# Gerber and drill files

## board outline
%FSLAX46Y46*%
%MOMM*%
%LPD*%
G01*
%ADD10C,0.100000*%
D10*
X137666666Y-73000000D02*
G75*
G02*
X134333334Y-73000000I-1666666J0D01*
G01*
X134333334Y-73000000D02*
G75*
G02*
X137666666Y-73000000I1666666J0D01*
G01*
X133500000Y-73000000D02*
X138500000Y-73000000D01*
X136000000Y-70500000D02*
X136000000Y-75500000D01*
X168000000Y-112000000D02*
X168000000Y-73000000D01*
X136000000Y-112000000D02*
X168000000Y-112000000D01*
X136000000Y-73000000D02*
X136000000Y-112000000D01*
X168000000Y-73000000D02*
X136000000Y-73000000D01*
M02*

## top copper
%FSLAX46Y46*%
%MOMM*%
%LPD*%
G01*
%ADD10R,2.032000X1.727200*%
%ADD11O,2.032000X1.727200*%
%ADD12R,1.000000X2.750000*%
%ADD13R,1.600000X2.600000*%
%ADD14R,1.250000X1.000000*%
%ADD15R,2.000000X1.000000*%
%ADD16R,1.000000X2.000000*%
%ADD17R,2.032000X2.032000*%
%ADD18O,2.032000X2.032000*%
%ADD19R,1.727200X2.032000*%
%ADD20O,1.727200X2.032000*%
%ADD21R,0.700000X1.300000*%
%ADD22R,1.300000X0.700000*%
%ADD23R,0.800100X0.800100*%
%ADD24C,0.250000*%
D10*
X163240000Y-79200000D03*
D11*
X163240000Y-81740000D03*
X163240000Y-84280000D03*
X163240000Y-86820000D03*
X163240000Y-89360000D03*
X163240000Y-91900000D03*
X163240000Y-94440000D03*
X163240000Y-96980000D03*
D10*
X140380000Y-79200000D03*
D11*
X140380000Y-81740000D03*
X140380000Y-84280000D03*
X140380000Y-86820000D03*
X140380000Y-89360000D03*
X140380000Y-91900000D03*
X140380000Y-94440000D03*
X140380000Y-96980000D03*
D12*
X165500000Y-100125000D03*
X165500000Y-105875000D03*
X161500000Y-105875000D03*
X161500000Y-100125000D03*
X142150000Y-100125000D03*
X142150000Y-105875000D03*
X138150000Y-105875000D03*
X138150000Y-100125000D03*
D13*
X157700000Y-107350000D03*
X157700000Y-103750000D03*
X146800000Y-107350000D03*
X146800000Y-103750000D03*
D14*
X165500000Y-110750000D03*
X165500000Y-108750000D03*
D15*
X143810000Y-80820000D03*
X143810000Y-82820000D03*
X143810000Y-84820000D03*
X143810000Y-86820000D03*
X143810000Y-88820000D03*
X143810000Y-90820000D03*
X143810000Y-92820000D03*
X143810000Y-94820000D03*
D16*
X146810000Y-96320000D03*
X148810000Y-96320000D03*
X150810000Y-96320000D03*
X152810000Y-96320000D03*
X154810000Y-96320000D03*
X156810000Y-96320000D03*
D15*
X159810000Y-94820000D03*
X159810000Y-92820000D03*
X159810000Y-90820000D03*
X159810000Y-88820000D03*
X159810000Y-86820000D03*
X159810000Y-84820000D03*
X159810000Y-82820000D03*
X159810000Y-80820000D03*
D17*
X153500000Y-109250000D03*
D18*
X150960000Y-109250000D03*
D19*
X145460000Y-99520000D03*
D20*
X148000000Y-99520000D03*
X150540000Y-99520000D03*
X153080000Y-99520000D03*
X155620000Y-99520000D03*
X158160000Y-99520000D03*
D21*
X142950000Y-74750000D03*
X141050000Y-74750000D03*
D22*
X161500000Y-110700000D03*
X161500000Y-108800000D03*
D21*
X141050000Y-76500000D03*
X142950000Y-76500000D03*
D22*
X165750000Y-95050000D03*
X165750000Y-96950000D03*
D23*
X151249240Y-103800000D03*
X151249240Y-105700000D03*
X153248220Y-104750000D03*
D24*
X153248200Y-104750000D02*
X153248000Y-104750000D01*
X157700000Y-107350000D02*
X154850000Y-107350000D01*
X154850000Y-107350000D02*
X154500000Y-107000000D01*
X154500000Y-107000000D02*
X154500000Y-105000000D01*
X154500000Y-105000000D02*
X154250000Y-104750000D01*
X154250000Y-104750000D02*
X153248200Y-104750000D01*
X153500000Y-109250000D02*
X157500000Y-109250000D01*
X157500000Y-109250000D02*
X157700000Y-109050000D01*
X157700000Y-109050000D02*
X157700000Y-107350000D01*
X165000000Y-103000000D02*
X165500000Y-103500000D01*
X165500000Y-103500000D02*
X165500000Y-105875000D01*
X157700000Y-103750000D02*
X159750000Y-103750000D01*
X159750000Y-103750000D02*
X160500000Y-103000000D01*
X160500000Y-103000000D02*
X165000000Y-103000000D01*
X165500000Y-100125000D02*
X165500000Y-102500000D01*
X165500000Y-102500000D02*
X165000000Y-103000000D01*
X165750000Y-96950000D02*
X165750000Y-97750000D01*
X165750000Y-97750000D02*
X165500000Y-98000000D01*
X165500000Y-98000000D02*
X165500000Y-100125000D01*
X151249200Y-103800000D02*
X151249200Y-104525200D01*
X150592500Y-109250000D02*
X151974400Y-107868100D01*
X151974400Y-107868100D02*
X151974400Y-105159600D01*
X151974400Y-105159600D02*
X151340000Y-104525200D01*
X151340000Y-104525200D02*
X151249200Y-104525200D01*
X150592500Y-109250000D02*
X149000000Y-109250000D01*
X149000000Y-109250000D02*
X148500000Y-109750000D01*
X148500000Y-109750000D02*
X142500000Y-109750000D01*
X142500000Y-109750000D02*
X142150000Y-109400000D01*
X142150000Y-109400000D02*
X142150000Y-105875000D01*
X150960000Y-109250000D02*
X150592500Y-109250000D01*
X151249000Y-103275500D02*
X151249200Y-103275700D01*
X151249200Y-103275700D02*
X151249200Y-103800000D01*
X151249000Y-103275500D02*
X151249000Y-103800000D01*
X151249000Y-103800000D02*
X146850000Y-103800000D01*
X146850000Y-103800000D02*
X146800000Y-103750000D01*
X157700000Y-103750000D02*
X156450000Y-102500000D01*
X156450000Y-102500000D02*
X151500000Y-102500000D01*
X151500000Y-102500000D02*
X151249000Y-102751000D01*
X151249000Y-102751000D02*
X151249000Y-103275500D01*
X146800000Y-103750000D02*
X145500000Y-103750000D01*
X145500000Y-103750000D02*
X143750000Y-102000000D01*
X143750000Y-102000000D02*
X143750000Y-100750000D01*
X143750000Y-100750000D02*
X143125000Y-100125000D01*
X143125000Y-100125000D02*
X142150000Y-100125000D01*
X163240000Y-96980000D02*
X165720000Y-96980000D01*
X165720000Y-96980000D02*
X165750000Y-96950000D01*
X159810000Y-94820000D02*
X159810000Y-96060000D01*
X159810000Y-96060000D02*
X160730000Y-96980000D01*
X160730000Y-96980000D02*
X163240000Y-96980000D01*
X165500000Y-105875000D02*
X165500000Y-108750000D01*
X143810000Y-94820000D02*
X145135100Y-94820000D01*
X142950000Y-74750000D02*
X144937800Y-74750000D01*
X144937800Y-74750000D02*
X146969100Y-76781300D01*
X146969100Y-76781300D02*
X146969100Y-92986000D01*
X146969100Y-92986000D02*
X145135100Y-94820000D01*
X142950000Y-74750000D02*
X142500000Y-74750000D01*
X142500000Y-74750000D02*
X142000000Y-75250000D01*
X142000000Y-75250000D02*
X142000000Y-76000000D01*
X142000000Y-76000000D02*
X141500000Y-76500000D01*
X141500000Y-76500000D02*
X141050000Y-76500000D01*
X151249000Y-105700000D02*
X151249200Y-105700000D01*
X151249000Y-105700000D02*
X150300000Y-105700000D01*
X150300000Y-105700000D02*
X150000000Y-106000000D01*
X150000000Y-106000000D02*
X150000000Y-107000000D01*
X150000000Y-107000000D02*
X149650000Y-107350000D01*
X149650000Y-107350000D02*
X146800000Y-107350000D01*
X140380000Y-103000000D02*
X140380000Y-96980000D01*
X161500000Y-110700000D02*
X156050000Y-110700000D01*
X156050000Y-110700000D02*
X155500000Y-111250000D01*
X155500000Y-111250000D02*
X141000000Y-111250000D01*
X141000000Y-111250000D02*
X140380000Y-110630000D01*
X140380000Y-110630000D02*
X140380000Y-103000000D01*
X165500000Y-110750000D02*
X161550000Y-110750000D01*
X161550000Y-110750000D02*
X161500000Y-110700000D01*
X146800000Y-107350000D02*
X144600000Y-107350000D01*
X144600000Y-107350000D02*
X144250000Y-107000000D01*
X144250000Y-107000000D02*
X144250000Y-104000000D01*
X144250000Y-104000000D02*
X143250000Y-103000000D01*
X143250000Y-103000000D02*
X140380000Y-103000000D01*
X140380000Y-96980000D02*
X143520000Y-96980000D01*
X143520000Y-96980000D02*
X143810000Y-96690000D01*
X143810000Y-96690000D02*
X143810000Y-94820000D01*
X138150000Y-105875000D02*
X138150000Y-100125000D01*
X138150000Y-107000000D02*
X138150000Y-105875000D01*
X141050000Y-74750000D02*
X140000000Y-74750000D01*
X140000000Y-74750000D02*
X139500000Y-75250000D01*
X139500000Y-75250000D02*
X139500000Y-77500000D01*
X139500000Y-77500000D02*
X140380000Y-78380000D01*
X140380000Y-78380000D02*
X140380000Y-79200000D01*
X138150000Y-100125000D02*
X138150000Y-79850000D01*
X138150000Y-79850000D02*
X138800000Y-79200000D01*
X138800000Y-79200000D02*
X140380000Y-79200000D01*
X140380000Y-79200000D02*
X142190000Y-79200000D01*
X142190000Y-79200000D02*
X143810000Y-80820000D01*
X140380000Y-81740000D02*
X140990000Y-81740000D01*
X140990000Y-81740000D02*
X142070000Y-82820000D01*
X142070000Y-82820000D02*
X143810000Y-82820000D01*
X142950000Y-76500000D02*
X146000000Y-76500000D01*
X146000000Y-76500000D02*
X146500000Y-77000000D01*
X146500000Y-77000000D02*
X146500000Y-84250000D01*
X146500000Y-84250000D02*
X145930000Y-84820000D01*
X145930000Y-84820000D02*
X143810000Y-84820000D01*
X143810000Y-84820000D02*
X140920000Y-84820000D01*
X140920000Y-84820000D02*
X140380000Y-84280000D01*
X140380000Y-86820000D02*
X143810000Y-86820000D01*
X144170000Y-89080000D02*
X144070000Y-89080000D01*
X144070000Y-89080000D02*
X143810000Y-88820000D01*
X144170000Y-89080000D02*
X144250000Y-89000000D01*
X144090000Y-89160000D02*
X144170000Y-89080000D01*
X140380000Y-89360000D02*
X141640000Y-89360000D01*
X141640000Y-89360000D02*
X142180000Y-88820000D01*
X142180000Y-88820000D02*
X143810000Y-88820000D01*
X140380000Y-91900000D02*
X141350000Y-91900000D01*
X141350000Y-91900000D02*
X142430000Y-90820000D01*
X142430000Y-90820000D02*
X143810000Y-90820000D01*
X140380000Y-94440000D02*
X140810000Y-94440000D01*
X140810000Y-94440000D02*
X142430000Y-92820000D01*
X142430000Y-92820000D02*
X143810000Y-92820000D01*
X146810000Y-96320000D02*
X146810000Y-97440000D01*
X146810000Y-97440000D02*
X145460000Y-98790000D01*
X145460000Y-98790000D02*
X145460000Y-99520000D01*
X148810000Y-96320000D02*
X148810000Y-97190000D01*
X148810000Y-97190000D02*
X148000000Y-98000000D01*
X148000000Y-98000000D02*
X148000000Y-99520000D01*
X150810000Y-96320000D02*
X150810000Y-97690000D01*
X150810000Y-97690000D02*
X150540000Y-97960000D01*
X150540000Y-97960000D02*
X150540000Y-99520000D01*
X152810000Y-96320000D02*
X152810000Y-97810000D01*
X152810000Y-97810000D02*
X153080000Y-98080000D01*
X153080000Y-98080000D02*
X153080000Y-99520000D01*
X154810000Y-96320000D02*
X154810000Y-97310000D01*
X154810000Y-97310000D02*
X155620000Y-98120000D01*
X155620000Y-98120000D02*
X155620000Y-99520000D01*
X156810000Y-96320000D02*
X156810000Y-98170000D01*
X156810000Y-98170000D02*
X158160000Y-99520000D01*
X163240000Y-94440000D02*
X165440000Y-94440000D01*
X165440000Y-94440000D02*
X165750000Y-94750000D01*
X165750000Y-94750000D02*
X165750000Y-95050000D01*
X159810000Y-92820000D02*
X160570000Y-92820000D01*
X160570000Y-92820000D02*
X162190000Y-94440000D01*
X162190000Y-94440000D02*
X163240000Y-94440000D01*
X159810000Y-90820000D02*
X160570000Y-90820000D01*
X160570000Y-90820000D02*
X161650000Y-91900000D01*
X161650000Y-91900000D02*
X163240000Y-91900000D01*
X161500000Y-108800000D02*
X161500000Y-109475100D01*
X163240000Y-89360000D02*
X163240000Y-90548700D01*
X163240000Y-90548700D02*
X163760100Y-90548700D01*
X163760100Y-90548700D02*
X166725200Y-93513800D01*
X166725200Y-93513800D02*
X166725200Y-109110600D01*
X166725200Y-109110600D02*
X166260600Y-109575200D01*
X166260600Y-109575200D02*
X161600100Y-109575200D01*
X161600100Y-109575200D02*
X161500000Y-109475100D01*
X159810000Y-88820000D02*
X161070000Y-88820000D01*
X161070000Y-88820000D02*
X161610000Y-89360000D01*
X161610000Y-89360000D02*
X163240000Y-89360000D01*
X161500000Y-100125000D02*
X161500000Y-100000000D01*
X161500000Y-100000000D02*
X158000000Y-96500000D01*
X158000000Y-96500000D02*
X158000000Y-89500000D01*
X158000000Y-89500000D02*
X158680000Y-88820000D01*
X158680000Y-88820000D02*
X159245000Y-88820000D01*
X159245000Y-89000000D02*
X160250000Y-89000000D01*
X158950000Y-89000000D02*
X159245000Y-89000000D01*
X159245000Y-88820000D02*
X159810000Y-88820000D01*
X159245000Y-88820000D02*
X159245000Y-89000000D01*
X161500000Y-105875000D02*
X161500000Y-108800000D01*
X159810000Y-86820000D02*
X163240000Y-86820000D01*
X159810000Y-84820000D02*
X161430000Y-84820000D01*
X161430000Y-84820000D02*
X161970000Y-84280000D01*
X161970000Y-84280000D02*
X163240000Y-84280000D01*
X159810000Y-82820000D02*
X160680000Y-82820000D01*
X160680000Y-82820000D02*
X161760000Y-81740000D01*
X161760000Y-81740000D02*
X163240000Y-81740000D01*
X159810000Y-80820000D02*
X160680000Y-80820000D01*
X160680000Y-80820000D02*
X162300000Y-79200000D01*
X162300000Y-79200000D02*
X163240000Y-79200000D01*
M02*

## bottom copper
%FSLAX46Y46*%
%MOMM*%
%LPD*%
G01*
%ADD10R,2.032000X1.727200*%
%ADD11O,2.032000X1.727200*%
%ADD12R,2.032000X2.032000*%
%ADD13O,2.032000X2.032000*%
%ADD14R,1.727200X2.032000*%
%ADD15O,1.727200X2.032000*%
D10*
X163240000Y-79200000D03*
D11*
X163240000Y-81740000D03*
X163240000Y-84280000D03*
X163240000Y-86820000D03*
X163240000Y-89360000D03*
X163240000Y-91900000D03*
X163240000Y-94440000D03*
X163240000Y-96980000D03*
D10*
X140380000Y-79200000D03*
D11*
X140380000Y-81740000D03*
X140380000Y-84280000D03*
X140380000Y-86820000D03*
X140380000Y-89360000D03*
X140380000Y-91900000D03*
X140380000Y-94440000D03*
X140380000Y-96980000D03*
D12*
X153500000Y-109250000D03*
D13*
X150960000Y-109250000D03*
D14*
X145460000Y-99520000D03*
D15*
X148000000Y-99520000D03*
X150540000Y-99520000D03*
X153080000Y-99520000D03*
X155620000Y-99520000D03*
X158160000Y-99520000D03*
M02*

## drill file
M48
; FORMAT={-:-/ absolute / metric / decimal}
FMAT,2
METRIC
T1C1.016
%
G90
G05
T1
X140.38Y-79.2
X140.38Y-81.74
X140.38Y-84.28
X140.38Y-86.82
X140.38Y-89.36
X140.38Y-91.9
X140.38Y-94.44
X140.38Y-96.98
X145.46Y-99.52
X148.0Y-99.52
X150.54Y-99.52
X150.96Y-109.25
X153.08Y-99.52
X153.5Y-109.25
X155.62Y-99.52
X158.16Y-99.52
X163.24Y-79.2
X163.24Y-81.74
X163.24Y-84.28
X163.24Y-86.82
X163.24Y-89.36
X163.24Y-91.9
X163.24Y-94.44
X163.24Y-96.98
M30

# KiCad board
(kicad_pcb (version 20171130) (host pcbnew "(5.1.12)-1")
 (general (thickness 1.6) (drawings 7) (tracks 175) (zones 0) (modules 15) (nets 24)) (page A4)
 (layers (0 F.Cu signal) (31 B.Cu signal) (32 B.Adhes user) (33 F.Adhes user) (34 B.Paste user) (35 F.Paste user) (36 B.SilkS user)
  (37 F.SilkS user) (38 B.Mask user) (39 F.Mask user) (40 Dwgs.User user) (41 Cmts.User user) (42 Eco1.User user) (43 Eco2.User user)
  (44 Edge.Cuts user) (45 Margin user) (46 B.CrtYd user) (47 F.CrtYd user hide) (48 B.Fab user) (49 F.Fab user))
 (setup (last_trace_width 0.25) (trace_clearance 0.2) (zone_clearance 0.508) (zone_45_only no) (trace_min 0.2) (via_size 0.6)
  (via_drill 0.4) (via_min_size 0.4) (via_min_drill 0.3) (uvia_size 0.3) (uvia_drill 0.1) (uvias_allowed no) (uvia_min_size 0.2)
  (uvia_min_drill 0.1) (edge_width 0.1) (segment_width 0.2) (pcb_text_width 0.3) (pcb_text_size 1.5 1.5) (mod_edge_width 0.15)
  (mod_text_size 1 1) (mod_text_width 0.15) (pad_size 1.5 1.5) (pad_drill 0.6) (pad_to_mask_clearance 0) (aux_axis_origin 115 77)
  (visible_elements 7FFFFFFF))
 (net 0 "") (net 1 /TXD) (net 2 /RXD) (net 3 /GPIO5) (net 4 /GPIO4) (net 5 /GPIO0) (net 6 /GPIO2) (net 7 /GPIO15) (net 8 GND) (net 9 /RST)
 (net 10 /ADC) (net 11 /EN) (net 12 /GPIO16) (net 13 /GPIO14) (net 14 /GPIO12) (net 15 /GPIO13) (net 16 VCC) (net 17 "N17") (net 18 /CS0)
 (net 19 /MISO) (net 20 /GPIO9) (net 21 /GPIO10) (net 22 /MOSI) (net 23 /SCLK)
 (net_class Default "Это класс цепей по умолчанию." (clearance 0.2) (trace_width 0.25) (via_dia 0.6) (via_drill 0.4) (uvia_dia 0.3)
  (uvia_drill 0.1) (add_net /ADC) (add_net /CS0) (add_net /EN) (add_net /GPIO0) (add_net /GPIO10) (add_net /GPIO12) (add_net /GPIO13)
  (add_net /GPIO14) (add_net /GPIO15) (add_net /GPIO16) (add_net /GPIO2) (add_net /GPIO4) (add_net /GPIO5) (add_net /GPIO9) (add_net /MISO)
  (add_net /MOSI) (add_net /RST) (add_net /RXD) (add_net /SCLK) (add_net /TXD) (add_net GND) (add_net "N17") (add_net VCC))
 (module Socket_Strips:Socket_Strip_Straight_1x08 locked (layer F.Cu) (at 163.24 79.2 270)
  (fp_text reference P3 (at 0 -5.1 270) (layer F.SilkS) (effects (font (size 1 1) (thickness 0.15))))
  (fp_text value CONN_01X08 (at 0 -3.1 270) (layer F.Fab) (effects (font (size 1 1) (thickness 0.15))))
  (pad 1 thru_hole rect (at 0 0 270) (size 1.7272 2.032) (drill 1.016) (layers *.Cu *.Mask F.SilkS) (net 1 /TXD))
  (pad 2 thru_hole oval (at 2.54 0 270) (size 1.7272 2.032) (drill 1.016) (layers *.Cu *.Mask F.SilkS) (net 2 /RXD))
  (pad 3 thru_hole oval (at 5.08 0 270) (size 1.7272 2.032) (drill 1.016) (layers *.Cu *.Mask F.SilkS) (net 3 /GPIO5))
  (pad 4 thru_hole oval (at 7.62 0 270) (size 1.7272 2.032) (drill 1.016) (layers *.Cu *.Mask F.SilkS) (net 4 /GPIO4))
  (pad 5 thru_hole oval (at 10.16 0 270) (size 1.7272 2.032) (drill 1.016) (layers *.Cu *.Mask F.SilkS) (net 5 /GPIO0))
  (pad 6 thru_hole oval (at 12.7 0 270) (size 1.7272 2.032) (drill 1.016) (layers *.Cu *.Mask F.SilkS) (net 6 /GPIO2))
  (pad 7 thru_hole oval (at 15.24 0 270) (size 1.7272 2.032) (drill 1.016) (layers *.Cu *.Mask F.SilkS) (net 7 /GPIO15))
  (pad 8 thru_hole oval (at 17.78 0 270) (size 1.7272 2.032) (drill 1.016) (layers *.Cu *.Mask F.SilkS) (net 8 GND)))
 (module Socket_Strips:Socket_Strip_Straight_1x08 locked (layer F.Cu) (at 140.38 79.2 270)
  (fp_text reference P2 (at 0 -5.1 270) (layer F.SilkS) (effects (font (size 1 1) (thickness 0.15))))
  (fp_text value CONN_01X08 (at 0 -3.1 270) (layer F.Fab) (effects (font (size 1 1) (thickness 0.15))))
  (pad 1 thru_hole rect (at 0 0 270) (size 1.7272 2.032) (drill 1.016) (layers *.Cu *.Mask F.SilkS) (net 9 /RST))
  (pad 2 thru_hole oval (at 2.54 0 270) (size 1.7272 2.032) (drill 1.016) (layers *.Cu *.Mask F.SilkS) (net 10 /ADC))
  (pad 3 thru_hole oval (at 5.08 0 270) (size 1.7272 2.032) (drill 1.016) (layers *.Cu *.Mask F.SilkS) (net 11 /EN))
  (pad 4 thru_hole oval (at 7.62 0 270) (size 1.7272 2.032) (drill 1.016) (layers *.Cu *.Mask F.SilkS) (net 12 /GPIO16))
  (pad 5 thru_hole oval (at 10.16 0 270) (size 1.7272 2.032) (drill 1.016) (layers *.Cu *.Mask F.SilkS) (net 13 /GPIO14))
  (pad 6 thru_hole oval (at 12.7 0 270) (size 1.7272 2.032) (drill 1.016) (layers *.Cu *.Mask F.SilkS) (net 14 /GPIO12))
  (pad 7 thru_hole oval (at 15.24 0 270) (size 1.7272 2.032) (drill 1.016) (layers *.Cu *.Mask F.SilkS) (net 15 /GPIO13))
  (pad 8 thru_hole oval (at 17.78 0 270) (size 1.7272 2.032) (drill 1.016) (layers *.Cu *.Mask F.SilkS) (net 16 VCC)))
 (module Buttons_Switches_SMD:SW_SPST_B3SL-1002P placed (layer F.Cu) (at 163.5 103 270)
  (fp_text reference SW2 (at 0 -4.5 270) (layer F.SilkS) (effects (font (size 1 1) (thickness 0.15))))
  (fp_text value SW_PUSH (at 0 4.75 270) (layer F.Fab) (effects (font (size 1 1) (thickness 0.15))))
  (pad 1 smd rect (at -2.875 -2 270) (size 2.75 1) (layers F.Cu F.Paste F.Mask) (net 8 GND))
  (pad 1 smd rect (at 2.875 -2 270) (size 2.75 1) (layers F.Cu F.Paste F.Mask) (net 8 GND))
  (pad 2 smd rect (at 2.875 2 270) (size 2.75 1) (layers F.Cu F.Paste F.Mask) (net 5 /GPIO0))
  (pad 2 smd rect (at -2.875 2 270) (size 2.75 1) (layers F.Cu F.Paste F.Mask) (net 5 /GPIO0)))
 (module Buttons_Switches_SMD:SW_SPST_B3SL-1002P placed (layer F.Cu) (at 140.15 103 270)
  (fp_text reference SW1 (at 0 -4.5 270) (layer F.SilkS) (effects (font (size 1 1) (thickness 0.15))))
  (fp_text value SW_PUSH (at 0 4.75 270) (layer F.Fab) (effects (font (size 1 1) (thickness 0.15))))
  (pad 1 smd rect (at -2.875 -2 270) (size 2.75 1) (layers F.Cu F.Paste F.Mask) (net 8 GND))
  (pad 1 smd rect (at 2.875 -2 270) (size 2.75 1) (layers F.Cu F.Paste F.Mask) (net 8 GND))
  (pad 2 smd rect (at 2.875 2 270) (size 2.75 1) (layers F.Cu F.Paste F.Mask) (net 9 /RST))
  (pad 2 smd rect (at -2.875 2 270) (size 2.75 1) (layers F.Cu F.Paste F.Mask) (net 9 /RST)))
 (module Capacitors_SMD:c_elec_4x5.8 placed (layer F.Cu) (at 157.7 105.55 90)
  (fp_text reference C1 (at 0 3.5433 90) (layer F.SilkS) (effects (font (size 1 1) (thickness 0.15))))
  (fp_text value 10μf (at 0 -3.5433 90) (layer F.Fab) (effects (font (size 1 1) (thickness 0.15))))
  (pad 1 smd rect (at -1.8 0 270) (size 2.6 1.6) (layers F.Cu F.Paste F.Mask) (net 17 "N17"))
  (pad 2 smd rect (at 1.8 0 270) (size 2.6 1.6) (layers F.Cu F.Paste F.Mask) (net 8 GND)))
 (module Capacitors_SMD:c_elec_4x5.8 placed (layer F.Cu) (at 146.8 105.55 90)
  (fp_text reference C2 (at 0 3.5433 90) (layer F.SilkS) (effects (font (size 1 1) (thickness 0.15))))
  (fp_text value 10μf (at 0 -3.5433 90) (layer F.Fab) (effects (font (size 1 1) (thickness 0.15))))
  (pad 1 smd rect (at -1.8 0 270) (size 2.6 1.6) (layers F.Cu F.Paste F.Mask) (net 16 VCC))
  (pad 2 smd rect (at 1.8 0 270) (size 2.6 1.6) (layers F.Cu F.Paste F.Mask) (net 8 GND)))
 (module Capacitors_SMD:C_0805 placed (layer F.Cu) (at 165.5 109.75 90)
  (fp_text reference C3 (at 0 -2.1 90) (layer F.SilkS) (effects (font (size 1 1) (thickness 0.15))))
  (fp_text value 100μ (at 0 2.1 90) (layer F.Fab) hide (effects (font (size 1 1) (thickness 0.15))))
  (pad 1 smd rect (at -1 0 90) (size 1 1.25) (layers F.Cu F.Paste F.Mask) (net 16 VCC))
  (pad 2 smd rect (at 1 0 90) (size 1 1.25) (layers F.Cu F.Paste F.Mask) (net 8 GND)))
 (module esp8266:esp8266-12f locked (layer F.Cu) (at 151.81 86.82)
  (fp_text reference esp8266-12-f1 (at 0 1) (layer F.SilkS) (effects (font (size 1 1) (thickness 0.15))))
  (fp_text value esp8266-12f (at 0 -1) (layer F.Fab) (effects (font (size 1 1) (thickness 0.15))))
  (pad 1 smd rect (at -8 -6) (size 2 1) (layers F.Cu F.Paste F.Mask) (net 9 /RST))
  (pad 2 smd rect (at -8 -4) (size 2 1) (layers F.Cu F.Paste F.Mask) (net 10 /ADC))
  (pad 3 smd rect (at -8 -2) (size 2 1) (layers F.Cu F.Paste F.Mask) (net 11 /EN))
  (pad 4 smd rect (at -8 0) (size 2 1) (layers F.Cu F.Paste F.Mask) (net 12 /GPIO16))
  (pad 5 smd rect (at -8 2) (size 2 1) (layers F.Cu F.Paste F.Mask) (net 13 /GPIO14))
  (pad 6 smd rect (at -8 4) (size 2 1) (layers F.Cu F.Paste F.Mask) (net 14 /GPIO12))
  (pad 7 smd rect (at -8 6) (size 2 1) (layers F.Cu F.Paste F.Mask) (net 15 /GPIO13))
  (pad 8 smd rect (at -8 8) (size 2 1) (layers F.Cu F.Paste F.Mask) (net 16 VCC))
  (pad 9 smd rect (at -5 9.5) (size 1 2) (layers F.Cu F.Paste F.Mask) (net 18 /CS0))
  (pad 10 smd rect (at -3 9.5) (size 1 2) (layers F.Cu F.Paste F.Mask) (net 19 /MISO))
  (pad 11 smd rect (at -1 9.5) (size 1 2) (layers F.Cu F.Paste F.Mask) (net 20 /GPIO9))
  (pad 12 smd rect (at 1 9.5) (size 1 2) (layers F.Cu F.Paste F.Mask) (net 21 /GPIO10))
  (pad 13 smd rect (at 3 9.5) (size 1 2) (layers F.Cu F.Paste F.Mask) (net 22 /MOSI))
  (pad 14 smd rect (at 5 9.5) (size 1 2) (layers F.Cu F.Paste F.Mask) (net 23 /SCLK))
  (pad 15 smd rect (at 8 8) (size 2 1) (layers F.Cu F.Paste F.Mask) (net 8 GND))
  (pad 16 smd rect (at 8 6) (size 2 1) (layers F.Cu F.Paste F.Mask) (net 7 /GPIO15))
  (pad 17 smd rect (at 8 4) (size 2 1) (layers F.Cu F.Paste F.Mask) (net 6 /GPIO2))
  (pad 18 smd rect (at 8 2) (size 2 1) (layers F.Cu F.Paste F.Mask) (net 5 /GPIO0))
  (pad 19 smd rect (at 8 0) (size 2 1) (layers F.Cu F.Paste F.Mask) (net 4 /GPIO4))
  (pad 20 smd rect (at 8 -2) (size 2 1) (layers F.Cu F.Paste F.Mask) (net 3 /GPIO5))
  (pad 21 smd rect (at 8 -4) (size 2 1) (layers F.Cu F.Paste F.Mask) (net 2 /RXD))
  (pad 22 smd rect (at 8 -6) (size 2 1) (layers F.Cu F.Paste F.Mask) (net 1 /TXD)))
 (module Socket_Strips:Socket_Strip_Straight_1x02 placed (layer F.Cu) (at 153.5 109.25 180)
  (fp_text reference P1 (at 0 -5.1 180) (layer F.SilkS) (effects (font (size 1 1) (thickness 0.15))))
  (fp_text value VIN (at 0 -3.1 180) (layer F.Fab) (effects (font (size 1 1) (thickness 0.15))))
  (pad 1 thru_hole rect (at 0 0 180) (size 2.032 2.032) (drill 1.016) (layers *.Cu *.Mask F.SilkS) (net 17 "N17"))
  (pad 2 thru_hole oval (at 2.54 0 180) (size 2.032 2.032) (drill 1.016) (layers *.Cu *.Mask F.SilkS) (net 8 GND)))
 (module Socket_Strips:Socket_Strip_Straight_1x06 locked (layer F.Cu) (at 145.46 99.52)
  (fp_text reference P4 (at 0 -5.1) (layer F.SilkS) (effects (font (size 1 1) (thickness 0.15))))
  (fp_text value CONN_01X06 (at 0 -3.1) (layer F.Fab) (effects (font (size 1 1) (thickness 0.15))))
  (pad 1 thru_hole rect (at 0 0) (size 1.7272 2.032) (drill 1.016) (layers *.Cu *.Mask F.SilkS) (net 18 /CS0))
  (pad 2 thru_hole oval (at 2.54 0) (size 1.7272 2.032) (drill 1.016) (layers *.Cu *.Mask F.SilkS) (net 19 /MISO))
  (pad 3 thru_hole oval (at 5.08 0) (size 1.7272 2.032) (drill 1.016) (layers *.Cu *.Mask F.SilkS) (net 20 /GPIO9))
  (pad 4 thru_hole oval (at 7.62 0) (size 1.7272 2.032) (drill 1.016) (layers *.Cu *.Mask F.SilkS) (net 21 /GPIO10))
  (pad 5 thru_hole oval (at 10.16 0) (size 1.7272 2.032) (drill 1.016) (layers *.Cu *.Mask F.SilkS) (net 22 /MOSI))
  (pad 6 thru_hole oval (at 12.7 0) (size 1.7272 2.032) (drill 1.016) (layers *.Cu *.Mask F.SilkS) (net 23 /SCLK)))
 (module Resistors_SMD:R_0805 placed (layer F.Cu) (at 142 74.75 180)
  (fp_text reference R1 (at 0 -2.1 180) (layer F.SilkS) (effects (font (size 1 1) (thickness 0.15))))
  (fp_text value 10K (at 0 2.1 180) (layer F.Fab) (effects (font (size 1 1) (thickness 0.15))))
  (pad 1 smd rect (at -0.95 0 180) (size 0.7 1.3) (layers F.Cu F.Paste F.Mask) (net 16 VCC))
  (pad 2 smd rect (at 0.95 0 180) (size 0.7 1.3) (layers F.Cu F.Paste F.Mask) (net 9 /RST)))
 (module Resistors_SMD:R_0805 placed (layer F.Cu) (at 161.5 109.75 90)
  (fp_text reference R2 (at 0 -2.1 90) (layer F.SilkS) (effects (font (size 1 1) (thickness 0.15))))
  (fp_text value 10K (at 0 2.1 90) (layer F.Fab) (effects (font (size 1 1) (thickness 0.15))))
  (pad 1 smd rect (at -0.95 0 90) (size 0.7 1.3) (layers F.Cu F.Paste F.Mask) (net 16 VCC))
  (pad 2 smd rect (at 0.95 0 90) (size 0.7 1.3) (layers F.Cu F.Paste F.Mask) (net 5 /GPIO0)))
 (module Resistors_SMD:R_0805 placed (layer F.Cu) (at 142 76.5)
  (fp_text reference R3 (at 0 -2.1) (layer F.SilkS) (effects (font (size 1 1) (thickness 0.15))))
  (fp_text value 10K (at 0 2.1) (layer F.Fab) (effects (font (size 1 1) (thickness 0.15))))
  (pad 1 smd rect (at -0.95 0) (size 0.7 1.3) (layers F.Cu F.Paste F.Mask) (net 16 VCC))
  (pad 2 smd rect (at 0.95 0) (size 0.7 1.3) (layers F.Cu F.Paste F.Mask) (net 11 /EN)))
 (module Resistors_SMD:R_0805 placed (layer F.Cu) (at 165.75 96 270)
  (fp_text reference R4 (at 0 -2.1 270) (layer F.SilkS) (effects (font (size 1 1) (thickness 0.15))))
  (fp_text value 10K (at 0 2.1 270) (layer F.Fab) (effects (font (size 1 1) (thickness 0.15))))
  (pad 1 smd rect (at -0.95 0 270) (size 0.7 1.3) (layers F.Cu F.Paste F.Mask) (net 7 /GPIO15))
  (pad 2 smd rect (at 0.95 0 270) (size 0.7 1.3) (layers F.Cu F.Paste F.Mask) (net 8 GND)))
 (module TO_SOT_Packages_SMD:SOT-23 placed (layer F.Cu) (at 152.25 104.75 270)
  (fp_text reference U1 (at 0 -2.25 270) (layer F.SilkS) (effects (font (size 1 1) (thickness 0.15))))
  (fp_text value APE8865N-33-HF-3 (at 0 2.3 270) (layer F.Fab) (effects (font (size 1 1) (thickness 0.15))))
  (pad 1 smd rect (at -0.95 1.00076 270) (size 0.8001 0.8001) (layers F.Cu F.Paste F.Mask) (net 8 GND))
  (pad 2 smd rect (at 0.95 1.00076 270) (size 0.8001 0.8001) (layers F.Cu F.Paste F.Mask) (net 16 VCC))
  (pad 3 smd rect (at 0 -0.99822 270) (size 0.8001 0.8001) (layers F.Cu F.Paste F.Mask) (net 17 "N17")))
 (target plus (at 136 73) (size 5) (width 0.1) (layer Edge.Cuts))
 (gr_line (start 168 112) (end 168 73) (angle 90) (layer Edge.Cuts) (width 0.1))
 (gr_line (start 136 112) (end 168 112) (angle 90) (layer Edge.Cuts) (width 0.1))
 (gr_line (start 136 73) (end 136 112) (angle 90) (layer Edge.Cuts) (width 0.1))
 (gr_line (start 168 73) (end 136 73) (angle 90) (layer Edge.Cuts) (width 0.1))
 (segment (start 153.2482 104.75) (end 153.248 104.75) (width 0.25) (layer F.Cu) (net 17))
 (segment (start 157.7 107.35) (end 154.85 107.35) (width 0.25) (layer F.Cu) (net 17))
 (segment (start 154.85 107.35) (end 154.5 107) (width 0.25) (layer F.Cu) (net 17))
 (segment (start 154.5 107) (end 154.5 105) (width 0.25) (layer F.Cu) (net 17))
 (segment (start 154.5 105) (end 154.25 104.75) (width 0.25) (layer F.Cu) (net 17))
 (segment (start 154.25 104.75) (end 153.2482 104.75) (width 0.25) (layer F.Cu) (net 17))
 (segment (start 153.5 109.25) (end 157.5 109.25) (width 0.25) (layer F.Cu) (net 17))
 (segment (start 157.5 109.25) (end 157.7 109.05) (width 0.25) (layer F.Cu) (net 17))
 (segment (start 157.7 109.05) (end 157.7 107.35) (width 0.25) (layer F.Cu) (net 17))
 (segment (start 165 103) (end 165.5 103.5) (width 0.25) (layer F.Cu) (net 8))
 (segment (start 165.5 103.5) (end 165.5 105.875) (width 0.25) (layer F.Cu) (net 8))
 (segment (start 157.7 103.75) (end 159.75 103.75) (width 0.25) (layer F.Cu) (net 8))
 (segment (start 159.75 103.75) (end 160.5 103) (width 0.25) (layer F.Cu) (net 8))
 (segment (start 160.5 103) (end 165 103) (width 0.25) (layer F.Cu) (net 8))
 (segment (start 165.5 100.125) (end 165.5 102.5) (width 0.25) (layer F.Cu) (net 8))
 (segment (start 165.5 102.5) (end 165 103) (width 0.25) (layer F.Cu) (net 8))
 (segment (start 165.75 96.95) (end 165.75 97.75) (width 0.25) (layer F.Cu) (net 8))
 (segment (start 165.75 97.75) (end 165.5 98) (width 0.25) (layer F.Cu) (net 8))
 (segment (start 165.5 98) (end 165.5 100.125) (width 0.25) (layer F.Cu) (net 8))
 (segment (start 151.2492 103.8) (end 151.2492 104.5252) (width 0.25) (layer F.Cu) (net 8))
 (segment (start 150.5925 109.25) (end 151.9744 107.8681) (width 0.25) (layer F.Cu) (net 8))
 (segment (start 151.9744 107.8681) (end 151.9744 105.1596) (width 0.25) (layer F.Cu) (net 8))
 (segment (start 151.9744 105.1596) (end 151.34 104.5252) (width 0.25) (layer F.Cu) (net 8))
 (segment (start 151.34 104.5252) (end 151.2492 104.5252) (width 0.25) (layer F.Cu) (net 8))
 (segment (start 150.5925 109.25) (end 149 109.25) (width 0.25) (layer F.Cu) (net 8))
 (segment (start 149 109.25) (end 148.5 109.75) (width 0.25) (layer F.Cu) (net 8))
 (segment (start 148.5 109.75) (end 142.5 109.75) (width 0.25) (layer F.Cu) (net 8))
 (segment (start 142.5 109.75) (end 142.15 109.4) (width 0.25) (layer F.Cu) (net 8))
 (segment (start 142.15 109.4) (end 142.15 105.875) (width 0.25) (layer F.Cu) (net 8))
 (segment (start 150.96 109.25) (end 150.5925 109.25) (width 0.25) (layer F.Cu) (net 8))
 (segment (start 151.249 103.2755) (end 151.2492 103.2757) (width 0.25) (layer F.Cu) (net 8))
 (segment (start 151.2492 103.2757) (end 151.2492 103.8) (width 0.25) (layer F.Cu) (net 8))
 (segment (start 151.249 103.2755) (end 151.249 103.8) (width 0.25) (layer F.Cu) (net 8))
 (segment (start 151.249 103.8) (end 146.85 103.8) (width 0.25) (layer F.Cu) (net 8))
 (segment (start 146.85 103.8) (end 146.8 103.75) (width 0.25) (layer F.Cu) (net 8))
 (segment (start 157.7 103.75) (end 156.45 102.5) (width 0.25) (layer F.Cu) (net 8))
 (segment (start 156.45 102.5) (end 151.5 102.5) (width 0.25) (layer F.Cu) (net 8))
 (segment (start 151.5 102.5) (end 151.249 102.751) (width 0.25) (layer F.Cu) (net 8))
 (segment (start 151.249 102.751) (end 151.249 103.2755) (width 0.25) (layer F.Cu) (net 8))
 (segment (start 146.8 103.75) (end 145.5 103.75) (width 0.25) (layer F.Cu) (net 8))
 (segment (start 145.5 103.75) (end 143.75 102) (width 0.25) (layer F.Cu) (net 8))
 (segment (start 143.75 102) (end 143.75 100.75) (width 0.25) (layer F.Cu) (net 8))
 (segment (start 143.75 100.75) (end 143.125 100.125) (width 0.25) (layer F.Cu) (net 8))
 (segment (start 143.125 100.125) (end 142.15 100.125) (width 0.25) (layer F.Cu) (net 8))
 (segment (start 163.24 96.98) (end 165.72 96.98) (width 0.25) (layer F.Cu) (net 8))
 (segment (start 165.72 96.98) (end 165.75 96.95) (width 0.25) (layer F.Cu) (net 8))
 (segment (start 159.81 94.82) (end 159.81 96.06) (width 0.25) (layer F.Cu) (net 8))
 (segment (start 159.81 96.06) (end 160.73 96.98) (width 0.25) (layer F.Cu) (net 8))
 (segment (start 160.73 96.98) (end 163.24 96.98) (width 0.25) (layer F.Cu) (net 8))
 (segment (start 165.5 105.875) (end 165.5 108.75) (width 0.25) (layer F.Cu) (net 8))
 (segment (start 143.81 94.82) (end 145.1351 94.82) (width 0.25) (layer F.Cu) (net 16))
 (segment (start 142.95 74.75) (end 144.9378 74.75) (width 0.25) (layer F.Cu) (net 16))
 (segment (start 144.9378 74.75) (end 146.9691 76.7813) (width 0.25) (layer F.Cu) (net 16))
 (segment (start 146.9691 76.7813) (end 146.9691 92.986) (width 0.25) (layer F.Cu) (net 16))
 (segment (start 146.9691 92.986) (end 145.1351 94.82) (width 0.25) (layer F.Cu) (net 16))
 (segment (start 142.95 74.75) (end 142.5 74.75) (width 0.25) (layer F.Cu) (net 16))
 (segment (start 142.5 74.75) (end 142 75.25) (width 0.25) (layer F.Cu) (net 16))
 (segment (start 142 75.25) (end 142 76) (width 0.25) (layer F.Cu) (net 16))
 (segment (start 142 76) (end 141.5 76.5) (width 0.25) (layer F.Cu) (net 16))
 (segment (start 141.5 76.5) (end 141.05 76.5) (width 0.25) (layer F.Cu) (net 16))
 (segment (start 151.249 105.7) (end 151.2492 105.7) (width 0.25) (layer F.Cu) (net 16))
 (segment (start 151.249 105.7) (end 150.3 105.7) (width 0.25) (layer F.Cu) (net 16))
 (segment (start 150.3 105.7) (end 150 106) (width 0.25) (layer F.Cu) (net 16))
 (segment (start 150 106) (end 150 107) (width 0.25) (layer F.Cu) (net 16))
 (segment (start 150 107) (end 149.65 107.35) (width 0.25) (layer F.Cu) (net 16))
 (segment (start 149.65 107.35) (end 146.8 107.35) (width 0.25) (layer F.Cu) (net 16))
 (segment (start 140.38 103) (end 140.38 96.98) (width 0.25) (layer F.Cu) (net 16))
 (segment (start 161.5 110.7) (end 156.05 110.7) (width 0.25) (layer F.Cu) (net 16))
 (segment (start 156.05 110.7) (end 155.5 111.25) (width 0.25) (layer F.Cu) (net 16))
 (segment (start 155.5 111.25) (end 141 111.25) (width 0.25) (layer F.Cu) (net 16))
 (segment (start 141 111.25) (end 140.38 110.63) (width 0.25) (layer F.Cu) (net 16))
 (segment (start 140.38 110.63) (end 140.38 103) (width 0.25) (layer F.Cu) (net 16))
 (segment (start 165.5 110.75) (end 161.55 110.75) (width 0.25) (layer F.Cu) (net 16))
 (segment (start 161.55 110.75) (end 161.5 110.7) (width 0.25) (layer F.Cu) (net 16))
 (segment (start 146.8 107.35) (end 144.6 107.35) (width 0.25) (layer F.Cu) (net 16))
 (segment (start 144.6 107.35) (end 144.25 107) (width 0.25) (layer F.Cu) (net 16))
 (segment (start 144.25 107) (end 144.25 104) (width 0.25) (layer F.Cu) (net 16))
 (segment (start 144.25 104) (end 143.25 103) (width 0.25) (layer F.Cu) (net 16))
 (segment (start 143.25 103) (end 140.38 103) (width 0.25) (layer F.Cu) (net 16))
 (segment (start 140.38 96.98) (end 143.52 96.98) (width 0.25) (layer F.Cu) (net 16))
 (segment (start 143.52 96.98) (end 143.81 96.69) (width 0.25) (layer F.Cu) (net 16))
 (segment (start 143.81 96.69) (end 143.81 94.82) (width 0.25) (layer F.Cu) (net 16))
 (segment (start 138.15 105.875) (end 138.15 100.125) (width 0.25) (layer F.Cu) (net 9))
 (segment (start 138.15 107) (end 138.15 105.875) (width 0.25) (layer F.Cu) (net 9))
 (segment (start 141.05 74.75) (end 140 74.75) (width 0.25) (layer F.Cu) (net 9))
 (segment (start 140 74.75) (end 139.5 75.25) (width 0.25) (layer F.Cu) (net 9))
 (segment (start 139.5 75.25) (end 139.5 77.5) (width 0.25) (layer F.Cu) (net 9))
 (segment (start 139.5 77.5) (end 140.38 78.38) (width 0.25) (layer F.Cu) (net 9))
 (segment (start 140.38 78.38) (end 140.38 79.2) (width 0.25) (layer F.Cu) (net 9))
 (segment (start 138.15 100.125) (end 138.15 79.85) (width 0.25) (layer F.Cu) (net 9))
 (segment (start 138.15 79.85) (end 138.8 79.2) (width 0.25) (layer F.Cu) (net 9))
 (segment (start 138.8 79.2) (end 140.38 79.2) (width 0.25) (layer F.Cu) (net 9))
 (segment (start 140.38 79.2) (end 142.19 79.2) (width 0.25) (layer F.Cu) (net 9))
 (segment (start 142.19 79.2) (end 143.81 80.82) (width 0.25) (layer F.Cu) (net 9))
 (segment (start 140.38 81.74) (end 140.99 81.74) (width 0.25) (layer F.Cu) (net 10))
 (segment (start 140.99 81.74) (end 142.07 82.82) (width 0.25) (layer F.Cu) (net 10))
 (segment (start 142.07 82.82) (end 143.81 82.82) (width 0.25) (layer F.Cu) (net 10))
 (segment (start 142.95 76.5) (end 146 76.5) (width 0.25) (layer F.Cu) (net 11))
 (segment (start 146 76.5) (end 146.5 77) (width 0.25) (layer F.Cu) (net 11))
 (segment (start 146.5 77) (end 146.5 84.25) (width 0.25) (layer F.Cu) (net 11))
 (segment (start 146.5 84.25) (end 145.93 84.82) (width 0.25) (layer F.Cu) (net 11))
 (segment (start 145.93 84.82) (end 143.81 84.82) (width 0.25) (layer F.Cu) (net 11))
 (segment (start 143.81 84.82) (end 140.92 84.82) (width 0.25) (layer F.Cu) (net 11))
 (segment (start 140.92 84.82) (end 140.38 84.28) (width 0.25) (layer F.Cu) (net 11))
 (segment (start 140.38 86.82) (end 143.81 86.82) (width 0.25) (layer F.Cu) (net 12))
 (segment (start 144.17 89.08) (end 144.07 89.08) (width 0.25) (layer F.Cu) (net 13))
 (segment (start 144.07 89.08) (end 143.81 88.82) (width 0.25) (layer F.Cu) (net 13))
 (segment (start 144.17 89.08) (end 144.25 89) (width 0.25) (layer F.Cu) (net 13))
 (segment (start 144.09 89.16) (end 144.17 89.08) (width 0.25) (layer F.Cu) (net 13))
 (segment (start 140.38 89.36) (end 141.64 89.36) (width 0.25) (layer F.Cu) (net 13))
 (segment (start 141.64 89.36) (end 142.18 88.82) (width 0.25) (layer F.Cu) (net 13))
 (segment (start 142.18 88.82) (end 143.81 88.82) (width 0.25) (layer F.Cu) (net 13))
 (segment (start 140.38 91.9) (end 141.35 91.9) (width 0.25) (layer F.Cu) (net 14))
 (segment (start 141.35 91.9) (end 142.43 90.82) (width 0.25) (layer F.Cu) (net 14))
 (segment (start 142.43 90.82) (end 143.81 90.82) (width 0.25) (layer F.Cu) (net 14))
 (segment (start 140.38 94.44) (end 140.81 94.44) (width 0.25) (layer F.Cu) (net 15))
 (segment (start 140.81 94.44) (end 142.43 92.82) (width 0.25) (layer F.Cu) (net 15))
 (segment (start 142.43 92.82) (end 143.81 92.82) (width 0.25) (layer F.Cu) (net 15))
 (segment (start 146.81 96.32) (end 146.81 97.44) (width 0.25) (layer F.Cu) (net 18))
 (segment (start 146.81 97.44) (end 145.46 98.79) (width 0.25) (layer F.Cu) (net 18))
 (segment (start 145.46 98.79) (end 145.46 99.52) (width 0.25) (layer F.Cu) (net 18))
 (segment (start 148.81 96.32) (end 148.81 97.19) (width 0.25) (layer F.Cu) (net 19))
 (segment (start 148.81 97.19) (end 148 98) (width 0.25) (layer F.Cu) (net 19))
 (segment (start 148 98) (end 148 99.52) (width 0.25) (layer F.Cu) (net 19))
 (segment (start 150.81 96.32) (end 150.81 97.69) (width 0.25) (layer F.Cu) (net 20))
 (segment (start 150.81 97.69) (end 150.54 97.96) (width 0.25) (layer F.Cu) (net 20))
 (segment (start 150.54 97.96) (end 150.54 99.52) (width 0.25) (layer F.Cu) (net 20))
 (segment (start 152.81 96.32) (end 152.81 97.81) (width 0.25) (layer F.Cu) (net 21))
 (segment (start 152.81 97.81) (end 153.08 98.08) (width 0.25) (layer F.Cu) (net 21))
 (segment (start 153.08 98.08) (end 153.08 99.52) (width 0.25) (layer F.Cu) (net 21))
 (segment (start 154.81 96.32) (end 154.81 97.31) (width 0.25) (layer F.Cu) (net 22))
 (segment (start 154.81 97.31) (end 155.62 98.12) (width 0.25) (layer F.Cu) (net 22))
 (segment (start 155.62 98.12) (end 155.62 99.52) (width 0.25) (layer F.Cu) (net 22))
 (segment (start 156.81 96.32) (end 156.81 98.17) (width 0.25) (layer F.Cu) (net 23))
 (segment (start 156.81 98.17) (end 158.16 99.52) (width 0.25) (layer F.Cu) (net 23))
 (segment (start 163.24 94.44) (end 165.44 94.44) (width 0.25) (layer F.Cu) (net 7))
 (segment (start 165.44 94.44) (end 165.75 94.75) (width 0.25) (layer F.Cu) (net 7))
 (segment (start 165.75 94.75) (end 165.75 95.05) (width 0.25) (layer F.Cu) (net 7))
 (segment (start 159.81 92.82) (end 160.57 92.82) (width 0.25) (layer F.Cu) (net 7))
 (segment (start 160.57 92.82) (end 162.19 94.44) (width 0.25) (layer F.Cu) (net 7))
 (segment (start 162.19 94.44) (end 163.24 94.44) (width 0.25) (layer F.Cu) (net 7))
 (segment (start 159.81 90.82) (end 160.57 90.82) (width 0.25) (layer F.Cu) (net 6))
 (segment (start 160.57 90.82) (end 161.65 91.9) (width 0.25) (layer F.Cu) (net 6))
 (segment (start 161.65 91.9) (end 163.24 91.9) (width 0.25) (layer F.Cu) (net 6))
 (segment (start 161.5 108.8) (end 161.5 109.4751) (width 0.25) (layer F.Cu) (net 5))
 (segment (start 163.24 89.36) (end 163.24 90.5487) (width 0.25) (layer F.Cu) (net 5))
 (segment (start 163.24 90.5487) (end 163.7601 90.5487) (width 0.25) (layer F.Cu) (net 5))
 (segment (start 163.7601 90.5487) (end 166.7252 93.5138) (width 0.25) (layer F.Cu) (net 5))
 (segment (start 166.7252 93.5138) (end 166.7252 109.1106) (width 0.25) (layer F.Cu) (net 5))
 (segment (start 166.7252 109.1106) (end 166.2606 109.5752) (width 0.25) (layer F.Cu) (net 5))
 (segment (start 166.2606 109.5752) (end 161.6001 109.5752) (width 0.25) (layer F.Cu) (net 5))
 (segment (start 161.6001 109.5752) (end 161.5 109.4751) (width 0.25) (layer F.Cu) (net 5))
 (segment (start 159.81 88.82) (end 161.07 88.82) (width 0.25) (layer F.Cu) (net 5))
 (segment (start 161.07 88.82) (end 161.61 89.36) (width 0.25) (layer F.Cu) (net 5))
 (segment (start 161.61 89.36) (end 163.24 89.36) (width 0.25) (layer F.Cu) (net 5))
 (segment (start 161.5 100.125) (end 161.5 100) (width 0.25) (layer F.Cu) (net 5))
 (segment (start 161.5 100) (end 158 96.5) (width 0.25) (layer F.Cu) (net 5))
 (segment (start 158 96.5) (end 158 89.5) (width 0.25) (layer F.Cu) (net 5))
 (segment (start 158 89.5) (end 158.68 88.82) (width 0.25) (layer F.Cu) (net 5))
 (segment (start 158.68 88.82) (end 159.245 88.82) (width 0.25) (layer F.Cu) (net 5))
 (segment (start 159.245 89) (end 160.25 89) (width 0.25) (layer F.Cu) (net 5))
 (segment (start 158.95 89) (end 159.245 89) (width 0.25) (layer F.Cu) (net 5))
 (segment (start 159.245 88.82) (end 159.81 88.82) (width 0.25) (layer F.Cu) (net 5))
 (segment (start 159.245 88.82) (end 159.245 89) (width 0.25) (layer F.Cu) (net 5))
 (segment (start 161.5 105.875) (end 161.5 108.8) (width 0.25) (layer F.Cu) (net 5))
 (segment (start 159.81 86.82) (end 163.24 86.82) (width 0.25) (layer F.Cu) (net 4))
 (segment (start 159.81 84.82) (end 161.43 84.82) (width 0.25) (layer F.Cu) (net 3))
 (segment (start 161.43 84.82) (end 161.97 84.28) (width 0.25) (layer F.Cu) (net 3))
 (segment (start 161.97 84.28) (end 163.24 84.28) (width 0.25) (layer F.Cu) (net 3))
 (segment (start 159.81 82.82) (end 160.68 82.82) (width 0.25) (layer F.Cu) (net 2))
 (segment (start 160.68 82.82) (end 161.76 81.74) (width 0.25) (layer F.Cu) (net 2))
 (segment (start 161.76 81.74) (end 163.24 81.74) (width 0.25) (layer F.Cu) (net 2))
 (segment (start 159.81 80.82) (end 160.68 80.82) (width 0.25) (layer F.Cu) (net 1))
 (segment (start 160.68 80.82) (end 162.3 79.2) (width 0.25) (layer F.Cu) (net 1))
 (segment (start 162.3 79.2) (end 163.24 79.2) (width 0.25) (layer F.Cu) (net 1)))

